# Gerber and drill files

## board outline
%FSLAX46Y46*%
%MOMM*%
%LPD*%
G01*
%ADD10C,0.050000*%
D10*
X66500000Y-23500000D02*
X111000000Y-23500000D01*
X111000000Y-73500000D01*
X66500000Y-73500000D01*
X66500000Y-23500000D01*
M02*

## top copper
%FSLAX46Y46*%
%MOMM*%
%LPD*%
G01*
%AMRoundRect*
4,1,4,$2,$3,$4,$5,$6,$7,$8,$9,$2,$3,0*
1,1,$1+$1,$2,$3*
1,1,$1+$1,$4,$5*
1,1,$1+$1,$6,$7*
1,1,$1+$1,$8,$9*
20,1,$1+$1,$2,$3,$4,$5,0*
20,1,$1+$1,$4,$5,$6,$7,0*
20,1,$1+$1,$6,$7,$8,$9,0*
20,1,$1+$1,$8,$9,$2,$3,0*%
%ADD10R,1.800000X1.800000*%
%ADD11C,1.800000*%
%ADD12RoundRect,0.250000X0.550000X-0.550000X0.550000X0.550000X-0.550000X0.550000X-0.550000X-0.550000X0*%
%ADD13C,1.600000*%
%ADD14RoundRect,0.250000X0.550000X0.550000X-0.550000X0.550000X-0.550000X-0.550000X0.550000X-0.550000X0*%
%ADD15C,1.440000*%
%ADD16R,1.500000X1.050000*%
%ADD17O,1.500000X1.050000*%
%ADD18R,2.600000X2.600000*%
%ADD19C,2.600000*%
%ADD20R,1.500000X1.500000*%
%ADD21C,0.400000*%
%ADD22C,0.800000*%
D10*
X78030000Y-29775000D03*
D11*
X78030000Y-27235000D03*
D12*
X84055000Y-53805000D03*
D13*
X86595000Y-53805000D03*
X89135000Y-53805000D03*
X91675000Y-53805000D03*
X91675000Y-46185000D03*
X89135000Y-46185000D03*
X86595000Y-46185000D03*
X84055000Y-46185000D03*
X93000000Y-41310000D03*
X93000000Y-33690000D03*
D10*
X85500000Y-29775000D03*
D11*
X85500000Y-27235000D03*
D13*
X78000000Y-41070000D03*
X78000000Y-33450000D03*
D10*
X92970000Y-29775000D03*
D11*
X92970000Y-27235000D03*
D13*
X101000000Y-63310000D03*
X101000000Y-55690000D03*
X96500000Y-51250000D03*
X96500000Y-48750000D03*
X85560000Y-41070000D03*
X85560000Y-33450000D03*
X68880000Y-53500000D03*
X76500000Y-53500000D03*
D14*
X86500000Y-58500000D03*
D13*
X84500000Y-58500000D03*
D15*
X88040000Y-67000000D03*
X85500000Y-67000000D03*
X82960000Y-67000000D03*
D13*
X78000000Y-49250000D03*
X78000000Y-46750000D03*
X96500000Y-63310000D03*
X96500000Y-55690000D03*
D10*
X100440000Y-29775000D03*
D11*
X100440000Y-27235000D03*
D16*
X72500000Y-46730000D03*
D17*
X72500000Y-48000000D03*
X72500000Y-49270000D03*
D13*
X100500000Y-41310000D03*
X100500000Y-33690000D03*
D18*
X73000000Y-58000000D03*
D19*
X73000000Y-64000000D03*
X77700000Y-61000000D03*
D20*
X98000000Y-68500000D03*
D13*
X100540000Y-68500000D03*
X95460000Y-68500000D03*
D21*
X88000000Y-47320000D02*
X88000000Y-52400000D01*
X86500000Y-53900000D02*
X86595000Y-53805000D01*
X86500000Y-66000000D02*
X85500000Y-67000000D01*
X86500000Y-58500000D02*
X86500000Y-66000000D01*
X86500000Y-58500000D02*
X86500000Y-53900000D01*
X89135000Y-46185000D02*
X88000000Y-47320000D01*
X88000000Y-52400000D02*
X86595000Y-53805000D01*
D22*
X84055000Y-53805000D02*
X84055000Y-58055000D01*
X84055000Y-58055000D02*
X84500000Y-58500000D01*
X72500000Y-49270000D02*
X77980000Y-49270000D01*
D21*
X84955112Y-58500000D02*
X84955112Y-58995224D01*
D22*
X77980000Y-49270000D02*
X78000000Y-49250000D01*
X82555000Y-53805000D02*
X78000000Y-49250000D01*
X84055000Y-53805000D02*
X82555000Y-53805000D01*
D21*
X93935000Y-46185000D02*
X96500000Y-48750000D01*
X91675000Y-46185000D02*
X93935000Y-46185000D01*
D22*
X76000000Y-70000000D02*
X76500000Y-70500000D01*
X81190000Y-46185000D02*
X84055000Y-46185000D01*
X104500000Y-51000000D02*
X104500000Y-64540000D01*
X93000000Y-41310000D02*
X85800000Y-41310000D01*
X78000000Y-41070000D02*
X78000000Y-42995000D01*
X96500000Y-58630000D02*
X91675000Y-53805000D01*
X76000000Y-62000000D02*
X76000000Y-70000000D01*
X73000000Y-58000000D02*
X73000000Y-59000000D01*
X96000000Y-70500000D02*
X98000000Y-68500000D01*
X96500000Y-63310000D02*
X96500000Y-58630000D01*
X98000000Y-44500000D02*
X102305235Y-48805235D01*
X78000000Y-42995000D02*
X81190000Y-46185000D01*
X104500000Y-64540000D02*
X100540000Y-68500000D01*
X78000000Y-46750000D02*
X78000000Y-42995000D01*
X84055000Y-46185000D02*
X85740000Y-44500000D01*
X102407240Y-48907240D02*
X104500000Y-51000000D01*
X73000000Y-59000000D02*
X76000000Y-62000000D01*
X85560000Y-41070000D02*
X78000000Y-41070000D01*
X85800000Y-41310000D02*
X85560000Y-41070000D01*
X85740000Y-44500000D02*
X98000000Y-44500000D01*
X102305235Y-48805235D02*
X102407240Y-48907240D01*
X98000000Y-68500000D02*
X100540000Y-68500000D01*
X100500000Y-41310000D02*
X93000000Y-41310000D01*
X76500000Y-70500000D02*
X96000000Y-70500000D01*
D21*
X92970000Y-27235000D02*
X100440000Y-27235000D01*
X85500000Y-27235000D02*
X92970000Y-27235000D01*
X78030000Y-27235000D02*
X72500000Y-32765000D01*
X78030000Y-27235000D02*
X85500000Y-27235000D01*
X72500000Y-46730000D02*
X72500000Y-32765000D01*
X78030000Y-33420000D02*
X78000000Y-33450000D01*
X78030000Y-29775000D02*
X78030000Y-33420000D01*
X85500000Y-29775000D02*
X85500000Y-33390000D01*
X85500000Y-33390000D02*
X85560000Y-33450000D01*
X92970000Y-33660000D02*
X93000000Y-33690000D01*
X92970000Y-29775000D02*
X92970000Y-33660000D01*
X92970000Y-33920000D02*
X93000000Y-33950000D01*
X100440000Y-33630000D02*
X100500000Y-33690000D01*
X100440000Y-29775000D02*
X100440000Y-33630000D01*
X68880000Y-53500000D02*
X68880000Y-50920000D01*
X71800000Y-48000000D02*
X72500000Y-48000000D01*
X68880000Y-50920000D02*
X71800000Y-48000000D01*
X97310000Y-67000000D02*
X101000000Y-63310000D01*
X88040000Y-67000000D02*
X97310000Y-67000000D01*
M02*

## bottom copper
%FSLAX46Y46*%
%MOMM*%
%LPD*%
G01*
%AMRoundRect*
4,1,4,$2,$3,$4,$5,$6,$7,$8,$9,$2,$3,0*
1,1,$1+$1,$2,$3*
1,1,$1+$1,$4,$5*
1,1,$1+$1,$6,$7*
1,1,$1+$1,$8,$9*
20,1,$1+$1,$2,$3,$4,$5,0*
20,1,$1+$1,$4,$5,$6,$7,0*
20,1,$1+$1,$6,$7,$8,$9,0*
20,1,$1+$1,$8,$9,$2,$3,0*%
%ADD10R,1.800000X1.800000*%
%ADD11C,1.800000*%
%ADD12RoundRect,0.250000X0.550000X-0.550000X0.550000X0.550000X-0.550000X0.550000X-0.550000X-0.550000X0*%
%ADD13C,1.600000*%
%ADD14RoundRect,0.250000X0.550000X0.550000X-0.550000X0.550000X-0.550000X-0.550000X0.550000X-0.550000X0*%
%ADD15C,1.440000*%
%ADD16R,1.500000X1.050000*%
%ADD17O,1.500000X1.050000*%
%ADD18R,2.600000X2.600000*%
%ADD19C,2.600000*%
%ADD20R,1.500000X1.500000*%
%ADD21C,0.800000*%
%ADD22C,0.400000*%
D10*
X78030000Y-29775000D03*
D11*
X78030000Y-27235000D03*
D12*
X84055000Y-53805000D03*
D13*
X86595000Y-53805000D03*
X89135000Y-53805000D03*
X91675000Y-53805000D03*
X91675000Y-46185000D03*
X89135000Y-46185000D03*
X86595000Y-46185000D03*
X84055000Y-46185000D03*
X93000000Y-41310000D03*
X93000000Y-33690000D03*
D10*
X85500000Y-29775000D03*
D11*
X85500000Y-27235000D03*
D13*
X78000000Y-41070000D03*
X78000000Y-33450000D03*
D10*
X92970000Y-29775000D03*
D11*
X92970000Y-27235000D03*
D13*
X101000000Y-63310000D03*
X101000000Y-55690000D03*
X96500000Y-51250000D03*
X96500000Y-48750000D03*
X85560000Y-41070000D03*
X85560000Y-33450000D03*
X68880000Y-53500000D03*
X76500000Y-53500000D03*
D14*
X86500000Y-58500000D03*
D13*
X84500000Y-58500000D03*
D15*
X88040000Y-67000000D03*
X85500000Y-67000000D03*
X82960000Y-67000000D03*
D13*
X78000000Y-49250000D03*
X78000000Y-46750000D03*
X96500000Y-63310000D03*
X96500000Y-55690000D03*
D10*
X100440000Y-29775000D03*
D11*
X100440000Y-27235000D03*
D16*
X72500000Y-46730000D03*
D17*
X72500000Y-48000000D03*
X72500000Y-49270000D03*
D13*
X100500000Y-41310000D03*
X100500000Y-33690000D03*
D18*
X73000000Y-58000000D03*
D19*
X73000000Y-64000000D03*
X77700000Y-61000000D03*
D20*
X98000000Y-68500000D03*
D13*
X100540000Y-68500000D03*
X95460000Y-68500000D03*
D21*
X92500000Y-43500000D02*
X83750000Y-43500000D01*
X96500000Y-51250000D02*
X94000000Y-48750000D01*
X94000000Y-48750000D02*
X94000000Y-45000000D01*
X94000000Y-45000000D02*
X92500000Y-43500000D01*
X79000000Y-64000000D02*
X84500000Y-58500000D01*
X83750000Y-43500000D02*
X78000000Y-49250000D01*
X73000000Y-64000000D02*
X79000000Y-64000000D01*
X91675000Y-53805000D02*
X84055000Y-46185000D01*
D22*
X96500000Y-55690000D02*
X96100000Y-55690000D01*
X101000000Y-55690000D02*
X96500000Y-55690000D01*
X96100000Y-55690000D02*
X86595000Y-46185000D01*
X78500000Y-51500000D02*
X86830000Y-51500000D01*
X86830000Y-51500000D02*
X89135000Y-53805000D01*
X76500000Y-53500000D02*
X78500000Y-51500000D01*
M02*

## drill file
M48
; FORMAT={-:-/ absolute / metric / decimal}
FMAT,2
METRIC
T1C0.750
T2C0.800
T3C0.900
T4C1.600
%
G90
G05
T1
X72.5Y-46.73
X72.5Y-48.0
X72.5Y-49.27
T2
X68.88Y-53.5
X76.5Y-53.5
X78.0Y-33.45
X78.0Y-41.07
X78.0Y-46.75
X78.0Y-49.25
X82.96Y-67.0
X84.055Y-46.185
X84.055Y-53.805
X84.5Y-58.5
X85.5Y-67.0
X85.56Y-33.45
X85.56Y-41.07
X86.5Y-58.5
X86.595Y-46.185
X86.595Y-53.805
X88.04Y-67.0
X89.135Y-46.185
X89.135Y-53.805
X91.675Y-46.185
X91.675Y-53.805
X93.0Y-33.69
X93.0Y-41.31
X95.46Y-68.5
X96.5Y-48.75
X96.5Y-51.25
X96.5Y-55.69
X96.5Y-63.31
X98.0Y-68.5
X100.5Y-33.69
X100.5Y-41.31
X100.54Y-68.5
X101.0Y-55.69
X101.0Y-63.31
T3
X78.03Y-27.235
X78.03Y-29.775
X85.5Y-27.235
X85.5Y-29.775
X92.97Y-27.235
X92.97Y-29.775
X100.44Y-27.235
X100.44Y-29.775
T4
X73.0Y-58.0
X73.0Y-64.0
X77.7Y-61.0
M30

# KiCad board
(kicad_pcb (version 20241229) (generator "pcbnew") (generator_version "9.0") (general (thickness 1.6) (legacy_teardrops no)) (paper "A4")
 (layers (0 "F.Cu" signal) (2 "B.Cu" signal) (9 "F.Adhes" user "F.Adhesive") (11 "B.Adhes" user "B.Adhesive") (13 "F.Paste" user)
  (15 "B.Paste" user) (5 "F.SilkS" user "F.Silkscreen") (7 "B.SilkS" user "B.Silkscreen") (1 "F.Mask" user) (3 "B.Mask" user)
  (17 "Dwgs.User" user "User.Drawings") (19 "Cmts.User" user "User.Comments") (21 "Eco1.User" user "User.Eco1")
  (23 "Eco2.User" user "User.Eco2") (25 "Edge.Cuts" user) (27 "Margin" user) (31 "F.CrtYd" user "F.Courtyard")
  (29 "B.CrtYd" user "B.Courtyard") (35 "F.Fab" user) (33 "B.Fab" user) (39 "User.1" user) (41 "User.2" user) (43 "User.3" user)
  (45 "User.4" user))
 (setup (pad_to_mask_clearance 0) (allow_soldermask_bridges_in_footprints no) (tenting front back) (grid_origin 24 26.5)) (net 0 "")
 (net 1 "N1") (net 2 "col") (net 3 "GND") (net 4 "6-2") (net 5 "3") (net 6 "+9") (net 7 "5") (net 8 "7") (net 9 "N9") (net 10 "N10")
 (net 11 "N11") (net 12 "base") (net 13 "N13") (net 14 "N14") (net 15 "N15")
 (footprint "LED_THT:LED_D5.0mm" (layer "F.Cu") (at 78.03 29.775 90)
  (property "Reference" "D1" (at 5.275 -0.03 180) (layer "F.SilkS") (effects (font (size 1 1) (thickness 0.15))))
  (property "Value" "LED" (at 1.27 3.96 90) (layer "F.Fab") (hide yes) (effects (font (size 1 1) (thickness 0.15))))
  (pad "1" thru_hole rect (at 0 0 90) (size 1.8 1.8) (drill 0.9) (layers "*.Cu" "*.Mask") (remove_unused_layers no) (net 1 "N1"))
  (pad "2" thru_hole circle (at 2.54 0 90) (size 1.8 1.8) (drill 0.9) (layers "*.Cu" "*.Mask") (remove_unused_layers no) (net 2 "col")))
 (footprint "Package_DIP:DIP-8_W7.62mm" (layer "F.Cu") (at 84.055 53.805 90)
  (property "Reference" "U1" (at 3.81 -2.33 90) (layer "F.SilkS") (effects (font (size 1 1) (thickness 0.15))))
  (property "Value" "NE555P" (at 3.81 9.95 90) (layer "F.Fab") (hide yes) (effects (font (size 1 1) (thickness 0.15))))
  (pad "1" thru_hole roundrect (at 0 0 90) (size 1.6 1.6) (drill 0.8) (layers "*.Cu" "*.Mask") (remove_unused_layers no)
   (roundrect_rratio 0.15625) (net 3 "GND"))
  (pad "2" thru_hole circle (at 0 2.54 90) (size 1.6 1.6) (drill 0.8) (layers "*.Cu" "*.Mask") (remove_unused_layers no) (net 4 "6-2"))
  (pad "3" thru_hole circle (at 0 5.08 90) (size 1.6 1.6) (drill 0.8) (layers "*.Cu" "*.Mask") (remove_unused_layers no) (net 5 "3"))
  (pad "4" thru_hole circle (at 0 7.62 90) (size 1.6 1.6) (drill 0.8) (layers "*.Cu" "*.Mask") (remove_unused_layers no) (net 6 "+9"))
  (pad "5" thru_hole circle (at 7.62 7.62 90) (size 1.6 1.6) (drill 0.8) (layers "*.Cu" "*.Mask") (remove_unused_layers no) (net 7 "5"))
  (pad "6" thru_hole circle (at 7.62 5.08 90) (size 1.6 1.6) (drill 0.8) (layers "*.Cu" "*.Mask") (remove_unused_layers no) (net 4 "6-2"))
  (pad "7" thru_hole circle (at 7.62 2.54 90) (size 1.6 1.6) (drill 0.8) (layers "*.Cu" "*.Mask") (remove_unused_layers no) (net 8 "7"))
  (pad "8" thru_hole circle (at 7.62 0 90) (size 1.6 1.6) (drill 0.8) (layers "*.Cu" "*.Mask") (remove_unused_layers no) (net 6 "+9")))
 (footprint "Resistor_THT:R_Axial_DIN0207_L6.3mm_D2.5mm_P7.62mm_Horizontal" (layer "F.Cu") (at 93 41.31 90)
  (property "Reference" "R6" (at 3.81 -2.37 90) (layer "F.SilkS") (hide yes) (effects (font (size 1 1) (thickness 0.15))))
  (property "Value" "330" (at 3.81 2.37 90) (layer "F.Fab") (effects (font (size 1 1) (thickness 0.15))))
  (pad "1" thru_hole circle (at 0 0 90) (size 1.6 1.6) (drill 0.8) (layers "*.Cu" "*.Mask") (remove_unused_layers no) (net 6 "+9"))
  (pad "2" thru_hole circle (at 7.62 0 90) (size 1.6 1.6) (drill 0.8) (layers "*.Cu" "*.Mask") (remove_unused_layers no) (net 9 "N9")))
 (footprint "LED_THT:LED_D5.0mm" (layer "F.Cu") (at 85.5 29.775 90)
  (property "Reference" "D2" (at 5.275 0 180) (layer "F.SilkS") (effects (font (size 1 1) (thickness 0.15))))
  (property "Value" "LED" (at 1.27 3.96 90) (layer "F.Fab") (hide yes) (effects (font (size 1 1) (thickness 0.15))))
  (pad "1" thru_hole rect (at 0 0 90) (size 1.8 1.8) (drill 0.9) (layers "*.Cu" "*.Mask") (remove_unused_layers no) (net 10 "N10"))
  (pad "2" thru_hole circle (at 2.54 0 90) (size 1.8 1.8) (drill 0.9) (layers "*.Cu" "*.Mask") (remove_unused_layers no) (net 2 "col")))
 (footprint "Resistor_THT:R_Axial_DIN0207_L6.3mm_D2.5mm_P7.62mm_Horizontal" (layer "F.Cu") (at 78 41.07 90)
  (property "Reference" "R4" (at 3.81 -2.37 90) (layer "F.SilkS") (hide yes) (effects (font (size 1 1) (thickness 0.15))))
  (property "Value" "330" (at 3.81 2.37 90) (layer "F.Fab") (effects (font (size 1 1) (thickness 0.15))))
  (pad "1" thru_hole circle (at 0 0 90) (size 1.6 1.6) (drill 0.8) (layers "*.Cu" "*.Mask") (remove_unused_layers no) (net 6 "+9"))
  (pad "2" thru_hole circle (at 7.62 0 90) (size 1.6 1.6) (drill 0.8) (layers "*.Cu" "*.Mask") (remove_unused_layers no) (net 1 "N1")))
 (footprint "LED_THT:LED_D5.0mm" (layer "F.Cu") (at 92.97 29.775 90)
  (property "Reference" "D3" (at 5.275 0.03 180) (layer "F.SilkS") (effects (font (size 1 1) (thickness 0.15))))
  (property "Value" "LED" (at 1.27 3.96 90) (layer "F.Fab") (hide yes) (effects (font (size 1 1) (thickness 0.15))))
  (pad "1" thru_hole rect (at 0 0 90) (size 1.8 1.8) (drill 0.9) (layers "*.Cu" "*.Mask") (remove_unused_layers no) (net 9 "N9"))
  (pad "2" thru_hole circle (at 2.54 0 90) (size 1.8 1.8) (drill 0.9) (layers "*.Cu" "*.Mask") (remove_unused_layers no) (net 2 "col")))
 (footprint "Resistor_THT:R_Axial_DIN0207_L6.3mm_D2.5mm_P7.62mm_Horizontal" (layer "F.Cu") (at 101 63.31 90)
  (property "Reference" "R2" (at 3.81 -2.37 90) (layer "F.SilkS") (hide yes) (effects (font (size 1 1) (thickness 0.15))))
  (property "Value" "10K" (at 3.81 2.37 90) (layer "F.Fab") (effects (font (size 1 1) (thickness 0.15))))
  (pad "1" thru_hole circle (at 0 0 90) (size 1.6 1.6) (drill 0.8) (layers "*.Cu" "*.Mask") (remove_unused_layers no) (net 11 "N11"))
  (pad "2" thru_hole circle (at 7.62 0 90) (size 1.6 1.6) (drill 0.8) (layers "*.Cu" "*.Mask") (remove_unused_layers no) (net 8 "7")))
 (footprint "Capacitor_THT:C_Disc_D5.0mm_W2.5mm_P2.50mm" (layer "F.Cu") (at 96.5 51.25 90)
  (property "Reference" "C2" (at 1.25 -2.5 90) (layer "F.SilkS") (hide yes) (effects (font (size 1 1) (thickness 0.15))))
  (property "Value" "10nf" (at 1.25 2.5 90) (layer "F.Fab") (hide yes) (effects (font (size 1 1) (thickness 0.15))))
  (pad "1" thru_hole circle (at 0 0 90) (size 1.6 1.6) (drill 0.8) (layers "*.Cu" "*.Mask") (remove_unused_layers no) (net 3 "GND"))
  (pad "2" thru_hole circle (at 2.5 0 90) (size 1.6 1.6) (drill 0.8) (layers "*.Cu" "*.Mask") (remove_unused_layers no) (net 7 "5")))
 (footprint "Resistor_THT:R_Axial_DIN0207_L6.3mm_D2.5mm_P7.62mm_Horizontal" (layer "F.Cu") (at 85.56 41.07 90)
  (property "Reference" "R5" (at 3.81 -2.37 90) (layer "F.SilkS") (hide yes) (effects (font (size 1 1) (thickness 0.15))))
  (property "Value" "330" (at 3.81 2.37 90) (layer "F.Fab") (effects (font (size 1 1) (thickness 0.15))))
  (pad "1" thru_hole circle (at 0 0 90) (size 1.6 1.6) (drill 0.8) (layers "*.Cu" "*.Mask") (remove_unused_layers no) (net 6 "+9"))
  (pad "2" thru_hole circle (at 7.62 0 90) (size 1.6 1.6) (drill 0.8) (layers "*.Cu" "*.Mask") (remove_unused_layers no) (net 10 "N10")))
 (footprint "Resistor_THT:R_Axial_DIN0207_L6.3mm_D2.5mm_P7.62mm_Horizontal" (layer "F.Cu") (at 68.88 53.5)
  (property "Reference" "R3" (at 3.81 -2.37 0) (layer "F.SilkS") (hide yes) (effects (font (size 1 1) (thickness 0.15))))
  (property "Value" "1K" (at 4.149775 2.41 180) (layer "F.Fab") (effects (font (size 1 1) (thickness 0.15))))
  (pad "1" thru_hole circle (at 0 0) (size 1.6 1.6) (drill 0.8) (layers "*.Cu" "*.Mask") (remove_unused_layers no) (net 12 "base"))
  (pad "2" thru_hole circle (at 7.62 0) (size 1.6 1.6) (drill 0.8) (layers "*.Cu" "*.Mask") (remove_unused_layers no) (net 5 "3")))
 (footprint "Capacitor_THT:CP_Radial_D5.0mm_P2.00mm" (layer "F.Cu") (at 86.5 58.5 180)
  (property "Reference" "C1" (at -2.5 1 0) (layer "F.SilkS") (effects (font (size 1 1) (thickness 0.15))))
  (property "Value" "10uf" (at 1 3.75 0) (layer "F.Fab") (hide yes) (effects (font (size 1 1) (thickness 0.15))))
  (pad "1" thru_hole roundrect (at 0 0 180) (size 1.6 1.6) (drill 0.8) (layers "*.Cu" "*.Mask") (remove_unused_layers no)
   (roundrect_rratio 0.15625) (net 4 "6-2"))
  (pad "2" thru_hole circle (at 2 0 180) (size 1.6 1.6) (drill 0.8) (layers "*.Cu" "*.Mask") (remove_unused_layers no) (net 3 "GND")))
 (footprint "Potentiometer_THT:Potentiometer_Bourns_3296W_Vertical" (layer "F.Cu") (at 88.04 67)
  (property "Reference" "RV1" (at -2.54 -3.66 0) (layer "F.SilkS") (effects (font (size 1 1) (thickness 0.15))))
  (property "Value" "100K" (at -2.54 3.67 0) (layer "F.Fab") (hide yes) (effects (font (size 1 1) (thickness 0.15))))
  (pad "1" thru_hole circle (at 0 0) (size 1.44 1.44) (drill 0.8) (layers "*.Cu" "*.Mask") (remove_unused_layers no) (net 11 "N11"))
  (pad "2" thru_hole circle (at -2.54 0) (size 1.44 1.44) (drill 0.8) (layers "*.Cu" "*.Mask") (remove_unused_layers no) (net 4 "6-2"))
  (pad "3" thru_hole circle (at -5.08 0) (size 1.44 1.44) (drill 0.8) (layers "*.Cu" "*.Mask") (remove_unused_layers no) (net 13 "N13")))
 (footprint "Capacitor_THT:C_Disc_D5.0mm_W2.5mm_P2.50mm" (layer "F.Cu") (at 78 49.25 90)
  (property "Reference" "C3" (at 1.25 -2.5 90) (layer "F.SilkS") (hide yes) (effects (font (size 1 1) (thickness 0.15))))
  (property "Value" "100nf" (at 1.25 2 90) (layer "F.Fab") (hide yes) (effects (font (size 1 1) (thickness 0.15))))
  (pad "1" thru_hole circle (at 0 0 90) (size 1.6 1.6) (drill 0.8) (layers "*.Cu" "*.Mask") (remove_unused_layers no) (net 3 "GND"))
  (pad "2" thru_hole circle (at 2.5 0 90) (size 1.6 1.6) (drill 0.8) (layers "*.Cu" "*.Mask") (remove_unused_layers no) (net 6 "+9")))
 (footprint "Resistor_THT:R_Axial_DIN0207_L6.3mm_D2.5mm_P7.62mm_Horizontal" (layer "F.Cu") (at 96.5 63.31 90)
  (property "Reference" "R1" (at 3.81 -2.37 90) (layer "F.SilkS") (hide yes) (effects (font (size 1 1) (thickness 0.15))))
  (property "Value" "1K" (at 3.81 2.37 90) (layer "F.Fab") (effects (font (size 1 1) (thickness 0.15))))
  (pad "1" thru_hole circle (at 0 0 90) (size 1.6 1.6) (drill 0.8) (layers "*.Cu" "*.Mask") (remove_unused_layers no) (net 6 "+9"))
  (pad "2" thru_hole circle (at 7.62 0 90) (size 1.6 1.6) (drill 0.8) (layers "*.Cu" "*.Mask") (remove_unused_layers no) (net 8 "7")))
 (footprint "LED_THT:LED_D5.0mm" (layer "F.Cu") (at 100.44 29.775 90)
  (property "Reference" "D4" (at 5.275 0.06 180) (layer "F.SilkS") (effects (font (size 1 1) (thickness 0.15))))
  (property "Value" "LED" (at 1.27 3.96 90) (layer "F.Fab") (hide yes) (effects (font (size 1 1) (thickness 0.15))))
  (pad "1" thru_hole rect (at 0 0 90) (size 1.8 1.8) (drill 0.9) (layers "*.Cu" "*.Mask") (remove_unused_layers no) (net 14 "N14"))
  (pad "2" thru_hole circle (at 2.54 0 90) (size 1.8 1.8) (drill 0.9) (layers "*.Cu" "*.Mask") (remove_unused_layers no) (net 2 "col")))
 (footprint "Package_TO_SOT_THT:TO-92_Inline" (layer "F.Cu") (at 72.5 46.73 -90)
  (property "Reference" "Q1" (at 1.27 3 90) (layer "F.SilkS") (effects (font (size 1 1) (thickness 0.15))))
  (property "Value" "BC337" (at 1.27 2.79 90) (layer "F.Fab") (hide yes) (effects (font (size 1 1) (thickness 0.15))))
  (pad "1" thru_hole rect (at 0 0 270) (size 1.05 1.5) (drill 0.75) (layers "*.Cu" "*.Mask") (remove_unused_layers no) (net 2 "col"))
  (pad "2" thru_hole oval (at 1.27 0 270) (size 1.05 1.5) (drill 0.75) (layers "*.Cu" "*.Mask") (remove_unused_layers no) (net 12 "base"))
  (pad "3" thru_hole oval (at 2.54 0 270) (size 1.05 1.5) (drill 0.75) (layers "*.Cu" "*.Mask") (remove_unused_layers no) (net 3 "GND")))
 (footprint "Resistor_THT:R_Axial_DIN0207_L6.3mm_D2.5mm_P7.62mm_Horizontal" (layer "F.Cu") (at 100.5 41.31 90)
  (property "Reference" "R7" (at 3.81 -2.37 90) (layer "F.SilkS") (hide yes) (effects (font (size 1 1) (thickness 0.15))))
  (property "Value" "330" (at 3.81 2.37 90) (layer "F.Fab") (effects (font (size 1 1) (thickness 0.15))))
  (pad "1" thru_hole circle (at 0 0 90) (size 1.6 1.6) (drill 0.8) (layers "*.Cu" "*.Mask") (remove_unused_layers no) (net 6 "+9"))
  (pad "2" thru_hole circle (at 7.62 0 90) (size 1.6 1.6) (drill 0.8) (layers "*.Cu" "*.Mask") (remove_unused_layers no) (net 14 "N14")))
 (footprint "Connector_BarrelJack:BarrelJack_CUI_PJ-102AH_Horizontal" (layer "F.Cu") (at 73 58)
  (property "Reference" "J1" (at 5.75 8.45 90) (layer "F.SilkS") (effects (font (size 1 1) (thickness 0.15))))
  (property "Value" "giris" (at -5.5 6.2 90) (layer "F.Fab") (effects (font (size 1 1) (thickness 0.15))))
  (pad "1" thru_hole rect (at 0 0) (size 2.6 2.6) (drill 1.6) (layers "*.Cu" "*.Mask") (remove_unused_layers no) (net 6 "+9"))
  (pad "2" thru_hole circle (at 0 6) (size 2.6 2.6) (drill 1.6) (layers "*.Cu" "*.Mask") (remove_unused_layers no) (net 3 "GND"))
  (pad "3" thru_hole circle (at 4.7 3) (size 2.6 2.6) (drill 1.6) (layers "*.Cu" "*.Mask") (remove_unused_layers no)))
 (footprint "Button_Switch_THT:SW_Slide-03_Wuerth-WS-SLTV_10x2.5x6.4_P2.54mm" (layer "F.Cu") (at 98 68.5 180)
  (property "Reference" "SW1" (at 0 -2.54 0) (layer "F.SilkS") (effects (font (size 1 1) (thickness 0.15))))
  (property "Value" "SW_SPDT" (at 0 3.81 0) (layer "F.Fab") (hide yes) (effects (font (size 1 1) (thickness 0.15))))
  (pad "1" thru_hole rect (at 0 0 180) (size 1.5 1.5) (drill 0.8) (layers "*.Cu" "*.Mask") (remove_unused_layers no) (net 6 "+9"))
  (pad "2" thru_hole circle (at -2.54 0 180) (size 1.6 1.6) (drill 0.8) (layers "*.Cu" "*.Mask") (remove_unused_layers no) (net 6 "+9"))
  (pad "3" thru_hole circle (at 2.54 0 180) (size 1.6 1.6) (drill 0.8) (layers "*.Cu" "*.Mask") (remove_unused_layers no) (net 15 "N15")))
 (gr_rect (start 66.5 23.5) (end 111 73.5) (stroke (width 0.05) (type default)) (fill no) (layer "Edge.Cuts"))
 (segment (start 88 47.32) (end 88 52.4) (width 0.4) (layer "F.Cu") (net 4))
 (segment (start 86.5 53.9) (end 86.595 53.805) (width 0.4) (layer "F.Cu") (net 4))
 (segment (start 86.5 66) (end 85.5 67) (width 0.4) (layer "F.Cu") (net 4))
 (segment (start 86.5 58.5) (end 86.5 66) (width 0.4) (layer "F.Cu") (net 4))
 (segment (start 86.5 58.5) (end 86.5 53.9) (width 0.4) (layer "F.Cu") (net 4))
 (segment (start 89.135 46.185) (end 88 47.32) (width 0.4) (layer "F.Cu") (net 4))
 (segment (start 88 52.4) (end 86.595 53.805) (width 0.4) (layer "F.Cu") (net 4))
 (segment (start 84.055 53.805) (end 84.055 58.055) (width 0.8) (layer "F.Cu") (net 3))
 (segment (start 84.055 58.055) (end 84.5 58.5) (width 0.8) (layer "F.Cu") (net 3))
 (segment (start 72.5 49.27) (end 77.98 49.27) (width 0.8) (layer "F.Cu") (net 3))
 (segment (start 84.955112 58.5) (end 84.955112 58.995224) (width 0.4) (layer "F.Cu") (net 3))
 (segment (start 77.98 49.27) (end 78 49.25) (width 0.8) (layer "F.Cu") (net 3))
 (segment (start 82.555 53.805) (end 78 49.25) (width 0.8) (layer "F.Cu") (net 3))
 (segment (start 84.055 53.805) (end 82.555 53.805) (width 0.8) (layer "F.Cu") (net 3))
 (segment (start 92.5 43.5) (end 83.75 43.5) (width 0.8) (layer "B.Cu") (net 3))
 (segment (start 96.5 51.25) (end 94 48.75) (width 0.8) (layer "B.Cu") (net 3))
 (segment (start 94 48.75) (end 94 45) (width 0.8) (layer "B.Cu") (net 3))
 (segment (start 94 45) (end 92.5 43.5) (width 0.8) (layer "B.Cu") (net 3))
 (segment (start 79 64) (end 84.5 58.5) (width 0.8) (layer "B.Cu") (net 3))
 (segment (start 83.75 43.5) (end 78 49.25) (width 0.8) (layer "B.Cu") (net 3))
 (segment (start 73 64) (end 79 64) (width 0.8) (layer "B.Cu") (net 3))
 (segment (start 93.935 46.185) (end 96.5 48.75) (width 0.4) (layer "F.Cu") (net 7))
 (segment (start 91.675 46.185) (end 93.935 46.185) (width 0.4) (layer "F.Cu") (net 7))
 (segment (start 76 70) (end 76.5 70.5) (width 0.8) (layer "F.Cu") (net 6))
 (segment (start 81.19 46.185) (end 84.055 46.185) (width 0.8) (layer "F.Cu") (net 6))
 (segment (start 104.5 51) (end 104.5 64.54) (width 0.8) (layer "F.Cu") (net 6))
 (segment (start 93 41.31) (end 85.8 41.31) (width 0.8) (layer "F.Cu") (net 6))
 (segment (start 78 41.07) (end 78 42.995) (width 0.8) (layer "F.Cu") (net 6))
 (segment (start 96.5 58.63) (end 91.675 53.805) (width 0.8) (layer "F.Cu") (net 6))
 (segment (start 76 62) (end 76 70) (width 0.8) (layer "F.Cu") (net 6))
 (segment (start 73 58) (end 73 59) (width 0.8) (layer "F.Cu") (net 6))
 (segment (start 96 70.5) (end 98 68.5) (width 0.8) (layer "F.Cu") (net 6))
 (segment (start 96.5 63.31) (end 96.5 58.63) (width 0.8) (layer "F.Cu") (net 6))
 (segment (start 98 44.5) (end 102.305235 48.805235) (width 0.8) (layer "F.Cu") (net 6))
 (segment (start 78 42.995) (end 81.19 46.185) (width 0.8) (layer "F.Cu") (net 6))
 (segment (start 104.5 64.54) (end 100.54 68.5) (width 0.8) (layer "F.Cu") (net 6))
 (segment (start 78 46.75) (end 78 42.995) (width 0.8) (layer "F.Cu") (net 6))
 (segment (start 84.055 46.185) (end 85.74 44.5) (width 0.8) (layer "F.Cu") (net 6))
 (segment (start 102.40724 48.90724) (end 104.5 51) (width 0.8) (layer "F.Cu") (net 6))
 (segment (start 73 59) (end 76 62) (width 0.8) (layer "F.Cu") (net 6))
 (segment (start 85.56 41.07) (end 78 41.07) (width 0.8) (layer "F.Cu") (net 6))
 (segment (start 85.8 41.31) (end 85.56 41.07) (width 0.8) (layer "F.Cu") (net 6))
 (segment (start 85.74 44.5) (end 98 44.5) (width 0.8) (layer "F.Cu") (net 6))
 (segment (start 102.305235 48.805235) (end 102.40724 48.90724) (width 0.8) (layer "F.Cu") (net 6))
 (segment (start 98 68.5) (end 100.54 68.5) (width 0.8) (layer "F.Cu") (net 6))
 (segment (start 100.5 41.31) (end 93 41.31) (width 0.8) (layer "F.Cu") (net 6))
 (segment (start 76.5 70.5) (end 96 70.5) (width 0.8) (layer "F.Cu") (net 6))
 (segment (start 91.675 53.805) (end 84.055 46.185) (width 0.8) (layer "B.Cu") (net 6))
 (segment (start 92.97 27.235) (end 100.44 27.235) (width 0.4) (layer "F.Cu") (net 2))
 (segment (start 85.5 27.235) (end 92.97 27.235) (width 0.4) (layer "F.Cu") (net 2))
 (segment (start 78.03 27.235) (end 72.5 32.765) (width 0.4) (layer "F.Cu") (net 2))
 (segment (start 78.03 27.235) (end 85.5 27.235) (width 0.4) (layer "F.Cu") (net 2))
 (segment (start 72.5 46.73) (end 72.5 32.765) (width 0.4) (layer "F.Cu") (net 2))
 (segment (start 78.03 33.42) (end 78 33.45) (width 0.4) (layer "F.Cu") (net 1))
 (segment (start 78.03 29.775) (end 78.03 33.42) (width 0.4) (layer "F.Cu") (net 1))
 (segment (start 85.5 29.775) (end 85.5 33.39) (width 0.4) (layer "F.Cu") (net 10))
 (segment (start 85.5 33.39) (end 85.56 33.45) (width 0.4) (layer "F.Cu") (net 10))
 (segment (start 92.97 33.66) (end 93 33.69) (width 0.4) (layer "F.Cu") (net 9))
 (segment (start 92.97 29.775) (end 92.97 33.66) (width 0.4) (layer "F.Cu") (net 9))
 (segment (start 92.97 33.92) (end 93 33.95) (width 0.4) (layer "F.Cu") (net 9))
 (segment (start 100.44 33.63) (end 100.5 33.69) (width 0.4) (layer "F.Cu") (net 14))
 (segment (start 100.44 29.775) (end 100.44 33.63) (width 0.4) (layer "F.Cu") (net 14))
 (segment (start 68.88 53.5) (end 68.88 50.92) (width 0.4) (layer "F.Cu") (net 12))
 (segment (start 71.8 48) (end 72.5 48) (width 0.4) (layer "F.Cu") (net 12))
 (segment (start 68.88 50.92) (end 71.8 48) (width 0.4) (layer "F.Cu") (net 12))
 (segment (start 96.5 55.69) (end 96.1 55.69) (width 0.4) (layer "B.Cu") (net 8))
 (segment (start 101 55.69) (end 96.5 55.69) (width 0.4) (layer "B.Cu") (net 8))
 (segment (start 96.1 55.69) (end 86.595 46.185) (width 0.4) (layer "B.Cu") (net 8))
 (segment (start 97.31 67) (end 101 63.31) (width 0.4) (layer "F.Cu") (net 11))
 (segment (start 88.04 67) (end 97.31 67) (width 0.4) (layer "F.Cu") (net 11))
 (segment (start 78.5 51.5) (end 86.83 51.5) (width 0.4) (layer "B.Cu") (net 5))
 (segment (start 86.83 51.5) (end 89.135 53.805) (width 0.4) (layer "B.Cu") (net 5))
 (segment (start 76.5 53.5) (end 78.5 51.5) (width 0.4) (layer "B.Cu") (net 5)))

